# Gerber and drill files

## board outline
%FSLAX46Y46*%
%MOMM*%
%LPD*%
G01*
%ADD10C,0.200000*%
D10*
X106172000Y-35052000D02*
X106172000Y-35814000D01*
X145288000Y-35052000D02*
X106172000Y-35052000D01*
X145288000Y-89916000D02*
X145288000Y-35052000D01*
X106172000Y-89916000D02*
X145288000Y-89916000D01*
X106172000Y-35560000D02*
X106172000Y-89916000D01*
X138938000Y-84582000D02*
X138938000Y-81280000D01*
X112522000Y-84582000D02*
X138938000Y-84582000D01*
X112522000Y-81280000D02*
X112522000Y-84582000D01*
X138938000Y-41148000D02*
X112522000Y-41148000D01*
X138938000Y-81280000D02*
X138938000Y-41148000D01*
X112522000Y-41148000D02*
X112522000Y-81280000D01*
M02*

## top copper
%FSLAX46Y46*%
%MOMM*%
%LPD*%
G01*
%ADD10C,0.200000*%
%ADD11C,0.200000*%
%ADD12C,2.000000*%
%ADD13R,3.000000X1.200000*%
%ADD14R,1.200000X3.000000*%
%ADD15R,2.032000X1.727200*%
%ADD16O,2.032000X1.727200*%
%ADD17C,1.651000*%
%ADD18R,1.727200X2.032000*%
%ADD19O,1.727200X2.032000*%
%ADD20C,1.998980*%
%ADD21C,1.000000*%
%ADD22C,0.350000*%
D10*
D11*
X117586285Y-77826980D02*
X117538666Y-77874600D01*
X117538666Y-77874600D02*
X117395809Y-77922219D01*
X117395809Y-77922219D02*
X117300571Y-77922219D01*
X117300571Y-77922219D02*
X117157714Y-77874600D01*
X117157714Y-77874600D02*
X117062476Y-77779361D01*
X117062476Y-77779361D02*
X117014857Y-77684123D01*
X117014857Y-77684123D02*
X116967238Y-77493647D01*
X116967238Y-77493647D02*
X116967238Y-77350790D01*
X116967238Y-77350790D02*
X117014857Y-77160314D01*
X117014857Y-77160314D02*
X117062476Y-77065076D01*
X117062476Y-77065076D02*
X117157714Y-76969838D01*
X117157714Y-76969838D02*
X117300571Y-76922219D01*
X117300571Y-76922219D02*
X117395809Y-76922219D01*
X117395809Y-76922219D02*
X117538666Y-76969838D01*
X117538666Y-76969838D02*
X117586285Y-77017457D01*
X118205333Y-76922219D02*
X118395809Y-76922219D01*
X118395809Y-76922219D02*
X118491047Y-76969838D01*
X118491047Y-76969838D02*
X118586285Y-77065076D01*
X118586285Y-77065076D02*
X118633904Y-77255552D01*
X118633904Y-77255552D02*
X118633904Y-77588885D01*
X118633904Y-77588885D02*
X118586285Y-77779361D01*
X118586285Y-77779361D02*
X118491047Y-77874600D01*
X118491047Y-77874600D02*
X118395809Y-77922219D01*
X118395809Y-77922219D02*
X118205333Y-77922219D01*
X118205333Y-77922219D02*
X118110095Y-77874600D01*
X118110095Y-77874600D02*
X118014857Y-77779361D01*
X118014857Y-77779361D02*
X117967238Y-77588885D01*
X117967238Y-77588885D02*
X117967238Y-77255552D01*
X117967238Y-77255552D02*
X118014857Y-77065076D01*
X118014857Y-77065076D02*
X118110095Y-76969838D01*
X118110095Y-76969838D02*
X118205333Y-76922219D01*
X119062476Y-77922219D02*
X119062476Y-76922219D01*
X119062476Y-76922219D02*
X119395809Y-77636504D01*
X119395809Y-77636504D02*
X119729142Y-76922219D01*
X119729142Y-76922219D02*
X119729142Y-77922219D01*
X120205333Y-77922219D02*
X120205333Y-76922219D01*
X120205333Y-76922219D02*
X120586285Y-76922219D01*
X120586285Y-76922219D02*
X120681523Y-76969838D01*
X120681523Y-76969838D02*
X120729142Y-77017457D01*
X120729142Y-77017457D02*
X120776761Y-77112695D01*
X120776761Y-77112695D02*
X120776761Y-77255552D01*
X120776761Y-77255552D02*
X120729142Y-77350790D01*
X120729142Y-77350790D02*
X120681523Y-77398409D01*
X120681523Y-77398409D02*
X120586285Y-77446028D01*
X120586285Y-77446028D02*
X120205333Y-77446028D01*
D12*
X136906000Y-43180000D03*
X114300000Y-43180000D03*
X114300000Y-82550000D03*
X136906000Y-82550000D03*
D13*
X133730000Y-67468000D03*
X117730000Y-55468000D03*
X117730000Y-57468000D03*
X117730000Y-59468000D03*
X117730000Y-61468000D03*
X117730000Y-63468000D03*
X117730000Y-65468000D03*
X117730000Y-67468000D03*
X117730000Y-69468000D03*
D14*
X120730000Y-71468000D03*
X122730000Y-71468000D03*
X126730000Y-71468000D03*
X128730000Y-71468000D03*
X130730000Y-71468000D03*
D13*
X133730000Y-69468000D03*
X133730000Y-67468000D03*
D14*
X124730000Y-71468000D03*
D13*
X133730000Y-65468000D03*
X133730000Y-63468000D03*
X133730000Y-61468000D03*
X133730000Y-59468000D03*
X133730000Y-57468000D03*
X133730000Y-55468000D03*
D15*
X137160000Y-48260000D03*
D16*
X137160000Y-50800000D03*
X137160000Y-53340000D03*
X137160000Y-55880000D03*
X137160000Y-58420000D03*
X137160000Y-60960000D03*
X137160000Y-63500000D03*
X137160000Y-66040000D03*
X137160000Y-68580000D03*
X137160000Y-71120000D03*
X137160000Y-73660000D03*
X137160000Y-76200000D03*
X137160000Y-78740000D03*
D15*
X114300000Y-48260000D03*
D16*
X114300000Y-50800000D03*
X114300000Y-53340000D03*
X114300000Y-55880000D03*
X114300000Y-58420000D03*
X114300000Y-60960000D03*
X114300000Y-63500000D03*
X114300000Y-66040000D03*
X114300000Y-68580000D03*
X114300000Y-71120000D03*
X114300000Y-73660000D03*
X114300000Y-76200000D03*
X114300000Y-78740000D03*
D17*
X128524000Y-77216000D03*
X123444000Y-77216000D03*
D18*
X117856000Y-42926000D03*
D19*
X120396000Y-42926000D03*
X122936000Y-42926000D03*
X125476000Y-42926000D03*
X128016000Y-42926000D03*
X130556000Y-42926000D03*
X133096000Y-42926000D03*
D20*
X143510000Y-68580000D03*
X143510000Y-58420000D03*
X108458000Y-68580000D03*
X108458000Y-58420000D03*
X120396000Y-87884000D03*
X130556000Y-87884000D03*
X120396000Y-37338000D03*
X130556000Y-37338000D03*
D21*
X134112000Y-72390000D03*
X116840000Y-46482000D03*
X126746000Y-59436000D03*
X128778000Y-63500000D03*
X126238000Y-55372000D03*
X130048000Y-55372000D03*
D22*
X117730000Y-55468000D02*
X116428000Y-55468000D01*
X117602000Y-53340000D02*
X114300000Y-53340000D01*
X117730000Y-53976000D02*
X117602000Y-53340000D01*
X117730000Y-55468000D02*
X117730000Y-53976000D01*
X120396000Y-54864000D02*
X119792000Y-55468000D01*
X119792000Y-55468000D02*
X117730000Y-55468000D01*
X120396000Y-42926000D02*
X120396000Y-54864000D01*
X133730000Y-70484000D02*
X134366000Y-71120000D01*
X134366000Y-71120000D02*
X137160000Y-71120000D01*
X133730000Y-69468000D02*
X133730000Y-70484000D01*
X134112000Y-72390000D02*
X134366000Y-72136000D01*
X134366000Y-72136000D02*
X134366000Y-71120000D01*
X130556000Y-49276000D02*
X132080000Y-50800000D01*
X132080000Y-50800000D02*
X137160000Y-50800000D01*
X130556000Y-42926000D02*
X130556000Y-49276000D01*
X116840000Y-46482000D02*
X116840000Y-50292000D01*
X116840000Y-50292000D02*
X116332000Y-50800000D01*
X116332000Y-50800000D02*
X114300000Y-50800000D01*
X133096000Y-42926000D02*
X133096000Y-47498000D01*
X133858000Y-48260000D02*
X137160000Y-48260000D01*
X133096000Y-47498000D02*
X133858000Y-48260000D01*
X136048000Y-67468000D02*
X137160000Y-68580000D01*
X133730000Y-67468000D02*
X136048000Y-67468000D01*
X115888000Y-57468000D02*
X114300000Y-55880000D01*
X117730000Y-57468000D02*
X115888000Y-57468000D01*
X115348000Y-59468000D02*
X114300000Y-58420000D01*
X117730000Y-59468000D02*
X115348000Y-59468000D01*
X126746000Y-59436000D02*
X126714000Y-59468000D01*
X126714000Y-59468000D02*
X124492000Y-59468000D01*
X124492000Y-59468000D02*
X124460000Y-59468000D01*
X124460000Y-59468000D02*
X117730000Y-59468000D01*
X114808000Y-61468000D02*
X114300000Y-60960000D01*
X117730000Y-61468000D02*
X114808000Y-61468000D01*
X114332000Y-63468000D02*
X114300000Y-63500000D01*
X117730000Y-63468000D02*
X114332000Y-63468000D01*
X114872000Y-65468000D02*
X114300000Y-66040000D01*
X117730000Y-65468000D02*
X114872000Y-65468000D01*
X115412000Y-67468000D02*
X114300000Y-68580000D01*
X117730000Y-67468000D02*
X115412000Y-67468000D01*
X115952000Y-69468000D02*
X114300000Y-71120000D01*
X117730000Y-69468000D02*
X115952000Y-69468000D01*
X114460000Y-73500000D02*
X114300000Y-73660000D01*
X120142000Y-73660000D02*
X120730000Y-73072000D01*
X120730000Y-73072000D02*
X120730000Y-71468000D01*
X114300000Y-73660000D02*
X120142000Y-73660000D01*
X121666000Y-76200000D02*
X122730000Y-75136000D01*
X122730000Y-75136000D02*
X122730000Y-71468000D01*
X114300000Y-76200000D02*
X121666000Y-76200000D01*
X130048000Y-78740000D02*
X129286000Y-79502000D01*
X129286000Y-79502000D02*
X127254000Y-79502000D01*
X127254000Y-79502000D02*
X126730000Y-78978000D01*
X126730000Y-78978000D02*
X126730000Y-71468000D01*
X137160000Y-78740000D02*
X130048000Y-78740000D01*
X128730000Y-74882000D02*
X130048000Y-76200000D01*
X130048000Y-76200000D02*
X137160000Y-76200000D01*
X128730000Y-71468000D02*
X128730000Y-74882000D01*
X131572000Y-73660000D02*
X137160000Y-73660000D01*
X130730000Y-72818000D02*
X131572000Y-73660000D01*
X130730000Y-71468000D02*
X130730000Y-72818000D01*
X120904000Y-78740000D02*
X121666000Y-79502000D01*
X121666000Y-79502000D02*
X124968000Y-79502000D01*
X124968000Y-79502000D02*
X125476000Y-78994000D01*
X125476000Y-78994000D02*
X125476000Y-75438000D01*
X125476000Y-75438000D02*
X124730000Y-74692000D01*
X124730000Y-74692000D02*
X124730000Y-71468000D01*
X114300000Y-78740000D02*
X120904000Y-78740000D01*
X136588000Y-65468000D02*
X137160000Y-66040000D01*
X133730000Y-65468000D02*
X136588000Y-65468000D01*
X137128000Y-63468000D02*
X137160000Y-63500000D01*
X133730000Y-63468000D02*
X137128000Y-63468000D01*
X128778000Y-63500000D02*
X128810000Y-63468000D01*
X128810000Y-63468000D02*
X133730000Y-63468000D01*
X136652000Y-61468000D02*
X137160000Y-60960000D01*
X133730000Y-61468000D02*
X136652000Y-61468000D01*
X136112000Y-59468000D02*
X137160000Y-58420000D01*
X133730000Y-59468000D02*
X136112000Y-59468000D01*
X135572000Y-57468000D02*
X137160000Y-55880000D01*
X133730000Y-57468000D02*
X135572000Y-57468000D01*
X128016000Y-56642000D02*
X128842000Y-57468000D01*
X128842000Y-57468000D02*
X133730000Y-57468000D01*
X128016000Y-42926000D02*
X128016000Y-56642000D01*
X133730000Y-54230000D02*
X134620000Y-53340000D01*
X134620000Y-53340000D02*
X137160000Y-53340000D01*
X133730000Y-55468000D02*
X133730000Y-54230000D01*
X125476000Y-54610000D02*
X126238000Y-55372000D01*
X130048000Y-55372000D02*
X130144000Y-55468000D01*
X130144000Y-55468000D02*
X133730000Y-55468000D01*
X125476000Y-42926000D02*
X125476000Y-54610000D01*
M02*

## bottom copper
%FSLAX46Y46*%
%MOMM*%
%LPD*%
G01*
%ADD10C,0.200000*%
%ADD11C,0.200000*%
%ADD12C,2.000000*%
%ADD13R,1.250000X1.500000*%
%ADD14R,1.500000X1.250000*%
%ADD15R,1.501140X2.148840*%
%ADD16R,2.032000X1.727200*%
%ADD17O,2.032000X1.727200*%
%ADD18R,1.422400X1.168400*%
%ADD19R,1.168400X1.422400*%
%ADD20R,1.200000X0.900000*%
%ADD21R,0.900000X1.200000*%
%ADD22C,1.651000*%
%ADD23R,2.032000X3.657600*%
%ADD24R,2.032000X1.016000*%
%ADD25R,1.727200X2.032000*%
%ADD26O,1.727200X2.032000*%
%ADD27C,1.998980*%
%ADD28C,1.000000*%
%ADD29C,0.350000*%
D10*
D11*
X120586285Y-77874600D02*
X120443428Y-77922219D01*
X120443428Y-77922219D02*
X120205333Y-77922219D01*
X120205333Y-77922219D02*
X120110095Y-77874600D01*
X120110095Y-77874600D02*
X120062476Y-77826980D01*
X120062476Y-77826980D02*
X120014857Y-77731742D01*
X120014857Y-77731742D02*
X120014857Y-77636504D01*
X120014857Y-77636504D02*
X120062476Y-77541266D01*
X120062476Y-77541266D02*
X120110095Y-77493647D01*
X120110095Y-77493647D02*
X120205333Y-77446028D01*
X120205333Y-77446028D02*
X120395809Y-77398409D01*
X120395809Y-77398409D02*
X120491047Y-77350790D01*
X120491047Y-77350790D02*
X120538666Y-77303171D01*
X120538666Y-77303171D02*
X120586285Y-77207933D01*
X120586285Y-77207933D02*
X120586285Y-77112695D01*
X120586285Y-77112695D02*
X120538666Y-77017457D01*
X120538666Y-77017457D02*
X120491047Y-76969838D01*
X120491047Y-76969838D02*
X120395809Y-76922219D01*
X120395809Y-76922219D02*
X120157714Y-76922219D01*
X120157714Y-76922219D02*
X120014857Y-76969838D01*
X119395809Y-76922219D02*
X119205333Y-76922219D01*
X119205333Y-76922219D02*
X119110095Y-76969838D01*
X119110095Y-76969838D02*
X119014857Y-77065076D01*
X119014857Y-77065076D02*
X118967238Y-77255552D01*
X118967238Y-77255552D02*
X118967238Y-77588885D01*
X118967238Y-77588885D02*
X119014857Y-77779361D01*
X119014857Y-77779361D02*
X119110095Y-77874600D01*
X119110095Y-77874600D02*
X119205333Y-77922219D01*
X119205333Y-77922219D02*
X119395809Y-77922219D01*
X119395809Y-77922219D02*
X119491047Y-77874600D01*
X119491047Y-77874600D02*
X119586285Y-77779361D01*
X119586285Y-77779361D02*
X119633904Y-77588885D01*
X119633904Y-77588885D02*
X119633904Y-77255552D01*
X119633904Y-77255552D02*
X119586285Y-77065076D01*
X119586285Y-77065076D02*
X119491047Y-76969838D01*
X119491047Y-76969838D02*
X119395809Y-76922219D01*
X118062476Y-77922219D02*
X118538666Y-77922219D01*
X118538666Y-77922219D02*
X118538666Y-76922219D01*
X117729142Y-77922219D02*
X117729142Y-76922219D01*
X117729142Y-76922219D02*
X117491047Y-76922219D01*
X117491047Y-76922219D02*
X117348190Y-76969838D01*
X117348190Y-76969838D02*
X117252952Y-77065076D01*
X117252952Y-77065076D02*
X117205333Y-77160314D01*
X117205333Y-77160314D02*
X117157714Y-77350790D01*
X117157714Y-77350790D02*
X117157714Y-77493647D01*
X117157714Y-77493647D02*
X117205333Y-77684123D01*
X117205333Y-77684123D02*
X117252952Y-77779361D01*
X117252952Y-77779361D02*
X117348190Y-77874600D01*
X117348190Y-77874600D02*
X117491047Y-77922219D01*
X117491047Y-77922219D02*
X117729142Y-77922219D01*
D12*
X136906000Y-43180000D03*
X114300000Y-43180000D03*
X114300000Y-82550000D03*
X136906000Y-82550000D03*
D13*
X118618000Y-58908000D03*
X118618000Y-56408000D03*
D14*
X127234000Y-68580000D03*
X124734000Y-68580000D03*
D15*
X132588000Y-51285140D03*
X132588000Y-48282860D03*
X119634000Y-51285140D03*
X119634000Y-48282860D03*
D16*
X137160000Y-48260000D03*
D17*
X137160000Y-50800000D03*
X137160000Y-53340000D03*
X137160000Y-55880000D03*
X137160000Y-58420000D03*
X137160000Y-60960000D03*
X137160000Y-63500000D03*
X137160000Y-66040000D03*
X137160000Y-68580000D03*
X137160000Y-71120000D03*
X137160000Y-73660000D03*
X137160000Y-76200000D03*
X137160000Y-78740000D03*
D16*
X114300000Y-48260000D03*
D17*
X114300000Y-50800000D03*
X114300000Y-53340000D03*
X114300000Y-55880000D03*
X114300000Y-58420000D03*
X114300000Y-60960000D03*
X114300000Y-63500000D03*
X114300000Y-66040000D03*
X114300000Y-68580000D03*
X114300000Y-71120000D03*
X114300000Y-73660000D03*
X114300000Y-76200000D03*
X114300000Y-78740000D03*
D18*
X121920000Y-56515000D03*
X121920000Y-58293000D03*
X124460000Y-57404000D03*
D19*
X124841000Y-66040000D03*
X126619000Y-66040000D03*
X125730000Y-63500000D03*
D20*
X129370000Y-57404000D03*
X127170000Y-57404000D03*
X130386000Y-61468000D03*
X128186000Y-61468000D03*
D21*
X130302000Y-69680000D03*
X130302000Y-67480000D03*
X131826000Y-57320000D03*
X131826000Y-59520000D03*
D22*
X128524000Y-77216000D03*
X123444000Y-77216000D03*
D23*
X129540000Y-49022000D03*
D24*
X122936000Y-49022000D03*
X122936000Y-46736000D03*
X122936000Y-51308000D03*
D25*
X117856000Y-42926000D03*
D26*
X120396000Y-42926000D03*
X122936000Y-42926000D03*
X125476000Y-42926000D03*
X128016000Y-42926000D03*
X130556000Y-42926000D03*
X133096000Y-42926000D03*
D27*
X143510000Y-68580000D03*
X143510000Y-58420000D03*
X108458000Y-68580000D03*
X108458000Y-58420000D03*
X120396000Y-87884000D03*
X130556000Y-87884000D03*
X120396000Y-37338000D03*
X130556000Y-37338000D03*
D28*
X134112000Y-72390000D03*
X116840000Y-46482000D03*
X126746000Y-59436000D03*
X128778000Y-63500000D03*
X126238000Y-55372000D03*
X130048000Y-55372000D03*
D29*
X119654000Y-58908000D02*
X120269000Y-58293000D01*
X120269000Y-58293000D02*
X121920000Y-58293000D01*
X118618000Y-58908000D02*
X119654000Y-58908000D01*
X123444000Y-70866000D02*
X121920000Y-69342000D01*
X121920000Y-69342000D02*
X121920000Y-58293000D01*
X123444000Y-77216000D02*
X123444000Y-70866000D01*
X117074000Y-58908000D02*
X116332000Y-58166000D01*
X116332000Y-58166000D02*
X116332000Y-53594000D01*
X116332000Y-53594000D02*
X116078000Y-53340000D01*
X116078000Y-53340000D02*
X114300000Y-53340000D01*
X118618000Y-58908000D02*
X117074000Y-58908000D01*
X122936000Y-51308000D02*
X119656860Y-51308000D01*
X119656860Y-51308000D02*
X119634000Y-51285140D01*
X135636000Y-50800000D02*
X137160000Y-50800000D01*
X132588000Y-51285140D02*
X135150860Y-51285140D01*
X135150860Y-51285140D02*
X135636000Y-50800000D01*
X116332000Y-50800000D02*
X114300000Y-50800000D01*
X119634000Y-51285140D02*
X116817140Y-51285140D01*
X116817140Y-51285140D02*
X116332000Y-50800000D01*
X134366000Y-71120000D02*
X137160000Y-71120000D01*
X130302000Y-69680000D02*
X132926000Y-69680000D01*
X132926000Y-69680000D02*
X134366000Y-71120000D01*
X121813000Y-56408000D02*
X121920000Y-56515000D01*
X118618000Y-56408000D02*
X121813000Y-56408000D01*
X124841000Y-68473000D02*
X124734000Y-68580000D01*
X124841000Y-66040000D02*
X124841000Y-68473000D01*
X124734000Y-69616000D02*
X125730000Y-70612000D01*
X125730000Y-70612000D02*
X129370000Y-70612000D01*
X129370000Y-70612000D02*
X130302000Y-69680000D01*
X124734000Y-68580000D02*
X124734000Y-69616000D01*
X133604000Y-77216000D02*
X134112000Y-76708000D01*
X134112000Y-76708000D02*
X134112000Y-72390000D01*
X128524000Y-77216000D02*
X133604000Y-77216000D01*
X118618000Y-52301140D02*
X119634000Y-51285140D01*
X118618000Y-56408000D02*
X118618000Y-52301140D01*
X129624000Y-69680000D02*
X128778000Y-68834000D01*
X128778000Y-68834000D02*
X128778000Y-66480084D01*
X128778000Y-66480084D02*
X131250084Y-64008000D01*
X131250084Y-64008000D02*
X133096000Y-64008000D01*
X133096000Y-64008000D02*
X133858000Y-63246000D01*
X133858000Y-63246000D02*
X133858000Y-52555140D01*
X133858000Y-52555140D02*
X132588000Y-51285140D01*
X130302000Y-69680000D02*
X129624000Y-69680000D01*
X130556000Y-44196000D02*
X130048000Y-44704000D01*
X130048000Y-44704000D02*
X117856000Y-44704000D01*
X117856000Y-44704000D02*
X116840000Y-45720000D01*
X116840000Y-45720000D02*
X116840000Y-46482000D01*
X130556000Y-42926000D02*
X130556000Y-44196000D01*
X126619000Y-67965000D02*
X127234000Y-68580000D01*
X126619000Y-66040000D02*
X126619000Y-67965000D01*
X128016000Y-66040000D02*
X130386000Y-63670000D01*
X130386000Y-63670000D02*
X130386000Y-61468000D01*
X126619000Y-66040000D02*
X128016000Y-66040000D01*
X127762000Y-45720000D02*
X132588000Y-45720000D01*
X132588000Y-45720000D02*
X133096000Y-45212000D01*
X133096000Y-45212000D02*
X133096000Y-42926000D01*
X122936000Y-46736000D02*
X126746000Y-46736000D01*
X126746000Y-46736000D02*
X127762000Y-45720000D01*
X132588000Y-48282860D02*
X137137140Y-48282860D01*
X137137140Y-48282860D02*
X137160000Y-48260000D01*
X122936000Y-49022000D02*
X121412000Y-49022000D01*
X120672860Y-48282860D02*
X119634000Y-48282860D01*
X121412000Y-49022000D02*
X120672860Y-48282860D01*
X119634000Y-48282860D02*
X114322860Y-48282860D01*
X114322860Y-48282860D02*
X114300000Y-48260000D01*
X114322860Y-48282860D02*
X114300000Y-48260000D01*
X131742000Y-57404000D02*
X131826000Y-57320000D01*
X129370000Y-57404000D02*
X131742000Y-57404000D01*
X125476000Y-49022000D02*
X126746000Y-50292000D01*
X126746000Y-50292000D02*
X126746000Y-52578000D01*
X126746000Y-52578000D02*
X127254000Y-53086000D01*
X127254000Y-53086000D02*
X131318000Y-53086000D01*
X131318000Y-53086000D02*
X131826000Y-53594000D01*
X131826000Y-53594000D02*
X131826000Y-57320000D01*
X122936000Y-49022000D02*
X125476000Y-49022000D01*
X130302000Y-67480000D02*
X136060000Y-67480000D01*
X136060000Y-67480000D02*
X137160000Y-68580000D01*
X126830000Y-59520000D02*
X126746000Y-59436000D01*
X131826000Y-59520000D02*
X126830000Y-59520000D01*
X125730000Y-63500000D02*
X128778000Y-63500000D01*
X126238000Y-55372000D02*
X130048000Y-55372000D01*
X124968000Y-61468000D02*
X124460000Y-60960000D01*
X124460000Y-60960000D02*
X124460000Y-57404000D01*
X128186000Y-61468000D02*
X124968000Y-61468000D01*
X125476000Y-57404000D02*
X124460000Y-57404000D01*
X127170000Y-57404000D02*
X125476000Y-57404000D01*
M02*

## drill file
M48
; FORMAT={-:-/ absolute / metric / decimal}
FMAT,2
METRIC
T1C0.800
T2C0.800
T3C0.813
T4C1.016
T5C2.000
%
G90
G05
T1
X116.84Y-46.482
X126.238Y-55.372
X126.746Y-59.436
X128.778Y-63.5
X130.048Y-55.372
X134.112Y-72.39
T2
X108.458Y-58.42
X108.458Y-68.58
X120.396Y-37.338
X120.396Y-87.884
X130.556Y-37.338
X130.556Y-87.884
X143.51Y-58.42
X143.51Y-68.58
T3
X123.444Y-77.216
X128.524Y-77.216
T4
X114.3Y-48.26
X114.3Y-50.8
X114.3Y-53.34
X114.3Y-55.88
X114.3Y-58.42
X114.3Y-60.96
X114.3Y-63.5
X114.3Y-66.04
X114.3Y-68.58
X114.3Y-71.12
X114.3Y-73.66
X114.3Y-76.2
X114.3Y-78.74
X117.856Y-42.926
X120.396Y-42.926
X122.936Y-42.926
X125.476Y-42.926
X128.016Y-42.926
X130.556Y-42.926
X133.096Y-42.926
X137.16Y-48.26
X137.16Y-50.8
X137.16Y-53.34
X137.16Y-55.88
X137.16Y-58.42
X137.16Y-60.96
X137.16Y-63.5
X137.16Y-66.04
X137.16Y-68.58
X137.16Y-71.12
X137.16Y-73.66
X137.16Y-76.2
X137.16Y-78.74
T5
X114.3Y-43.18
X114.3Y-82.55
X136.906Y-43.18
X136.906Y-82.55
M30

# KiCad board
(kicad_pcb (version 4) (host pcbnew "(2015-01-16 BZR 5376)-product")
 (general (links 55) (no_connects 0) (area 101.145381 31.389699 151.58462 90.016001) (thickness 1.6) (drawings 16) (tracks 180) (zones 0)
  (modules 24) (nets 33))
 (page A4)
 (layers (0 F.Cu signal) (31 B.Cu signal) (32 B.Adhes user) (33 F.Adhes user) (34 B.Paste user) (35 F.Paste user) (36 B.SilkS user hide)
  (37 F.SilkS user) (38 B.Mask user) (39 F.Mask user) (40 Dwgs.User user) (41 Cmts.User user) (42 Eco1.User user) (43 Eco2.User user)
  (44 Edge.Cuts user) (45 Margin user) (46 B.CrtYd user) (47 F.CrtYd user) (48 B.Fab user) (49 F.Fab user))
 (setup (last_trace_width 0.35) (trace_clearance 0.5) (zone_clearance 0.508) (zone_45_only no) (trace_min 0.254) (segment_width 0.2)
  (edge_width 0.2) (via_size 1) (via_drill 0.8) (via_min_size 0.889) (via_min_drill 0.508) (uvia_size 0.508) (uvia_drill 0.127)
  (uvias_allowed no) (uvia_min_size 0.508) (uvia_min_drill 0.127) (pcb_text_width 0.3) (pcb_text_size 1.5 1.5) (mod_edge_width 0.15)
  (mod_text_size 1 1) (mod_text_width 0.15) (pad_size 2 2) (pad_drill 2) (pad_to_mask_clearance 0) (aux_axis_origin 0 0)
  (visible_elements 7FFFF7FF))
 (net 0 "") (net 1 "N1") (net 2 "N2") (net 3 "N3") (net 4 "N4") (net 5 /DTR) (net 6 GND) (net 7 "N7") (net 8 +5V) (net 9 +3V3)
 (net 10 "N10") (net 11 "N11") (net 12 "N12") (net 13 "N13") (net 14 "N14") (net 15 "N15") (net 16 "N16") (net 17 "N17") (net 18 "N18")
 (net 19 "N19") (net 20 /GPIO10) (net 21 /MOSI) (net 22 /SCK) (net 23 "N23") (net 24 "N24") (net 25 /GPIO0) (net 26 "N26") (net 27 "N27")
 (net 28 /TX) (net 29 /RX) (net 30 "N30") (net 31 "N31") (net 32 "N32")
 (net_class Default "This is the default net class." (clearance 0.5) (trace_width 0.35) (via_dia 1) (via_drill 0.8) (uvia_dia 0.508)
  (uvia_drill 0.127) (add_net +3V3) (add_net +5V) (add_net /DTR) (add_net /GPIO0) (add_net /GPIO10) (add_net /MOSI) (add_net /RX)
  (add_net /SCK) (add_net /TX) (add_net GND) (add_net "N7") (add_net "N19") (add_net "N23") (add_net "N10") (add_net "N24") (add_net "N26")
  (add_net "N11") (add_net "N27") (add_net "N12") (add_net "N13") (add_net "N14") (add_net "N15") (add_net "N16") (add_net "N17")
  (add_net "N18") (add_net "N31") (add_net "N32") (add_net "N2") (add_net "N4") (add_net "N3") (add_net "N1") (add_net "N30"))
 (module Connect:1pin (layer F.Cu) (at 136.906 43.18)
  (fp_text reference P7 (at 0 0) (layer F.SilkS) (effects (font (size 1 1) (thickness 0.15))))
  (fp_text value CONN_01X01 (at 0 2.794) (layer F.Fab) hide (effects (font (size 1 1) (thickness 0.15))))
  (pad 1 thru_hole circle (at 0 0) (size 2 2) (drill 2) (layers *.Cu *.Mask F.SilkS) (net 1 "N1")))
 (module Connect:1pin (layer F.Cu) (at 114.3 43.18)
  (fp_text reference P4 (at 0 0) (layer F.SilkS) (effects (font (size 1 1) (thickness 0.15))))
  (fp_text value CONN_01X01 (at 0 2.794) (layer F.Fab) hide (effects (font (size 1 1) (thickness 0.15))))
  (pad 1 thru_hole circle (at 0 0) (size 2 2) (drill 2) (layers *.Cu *.Mask F.SilkS) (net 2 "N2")))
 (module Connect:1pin (layer F.Cu) (at 114.3 82.55)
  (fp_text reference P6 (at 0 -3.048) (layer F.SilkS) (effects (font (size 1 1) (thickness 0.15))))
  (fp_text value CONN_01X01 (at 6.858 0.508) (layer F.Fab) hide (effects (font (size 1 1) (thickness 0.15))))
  (pad 1 thru_hole circle (at 0 0) (size 2 2) (drill 2) (layers *.Cu *.Mask F.SilkS) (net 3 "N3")))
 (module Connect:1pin (layer F.Cu) (at 136.906 82.55)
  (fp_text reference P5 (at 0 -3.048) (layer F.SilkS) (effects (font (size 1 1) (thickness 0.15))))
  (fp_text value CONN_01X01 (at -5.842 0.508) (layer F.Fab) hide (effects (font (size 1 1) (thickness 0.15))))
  (pad 1 thru_hole circle (at 0 0) (size 2 2) (drill 2) (layers *.Cu *.Mask F.SilkS) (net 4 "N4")))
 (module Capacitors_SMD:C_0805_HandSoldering (layer B.Cu) (at 118.618 57.658 90)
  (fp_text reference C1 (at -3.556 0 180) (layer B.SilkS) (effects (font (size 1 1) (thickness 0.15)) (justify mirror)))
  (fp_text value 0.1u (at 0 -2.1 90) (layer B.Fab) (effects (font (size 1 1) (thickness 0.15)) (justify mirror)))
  (pad 1 smd rect (at -1.25 0 90) (size 1.5 1.25) (layers B.Cu B.Paste B.Mask) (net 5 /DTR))
  (pad 2 smd rect (at 1.25 0 90) (size 1.5 1.25) (layers B.Cu B.Paste B.Mask) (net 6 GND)))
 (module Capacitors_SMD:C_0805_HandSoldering (layer B.Cu) (at 125.984 68.58 180)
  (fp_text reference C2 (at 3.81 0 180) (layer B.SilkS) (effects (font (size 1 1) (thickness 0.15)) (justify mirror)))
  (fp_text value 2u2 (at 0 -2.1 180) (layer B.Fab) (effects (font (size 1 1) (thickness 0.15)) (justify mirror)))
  (pad 1 smd rect (at -1.25 0 180) (size 1.5 1.25) (layers B.Cu B.Paste B.Mask) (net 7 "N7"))
  (pad 2 smd rect (at 1.25 0 180) (size 1.5 1.25) (layers B.Cu B.Paste B.Mask) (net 6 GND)))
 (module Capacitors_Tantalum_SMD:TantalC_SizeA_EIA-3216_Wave (layer B.Cu) (at 132.588 49.784 270)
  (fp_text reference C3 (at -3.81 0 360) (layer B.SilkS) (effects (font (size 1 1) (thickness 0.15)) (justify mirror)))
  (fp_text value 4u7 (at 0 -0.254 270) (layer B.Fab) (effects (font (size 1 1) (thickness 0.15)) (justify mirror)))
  (pad 2 smd rect (at 1.50114 0 270) (size 2.14884 1.50114) (layers B.Cu B.Paste B.Mask) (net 6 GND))
  (pad 1 smd rect (at -1.50114 0 270) (size 2.14884 1.50114) (layers B.Cu B.Paste B.Mask) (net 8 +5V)))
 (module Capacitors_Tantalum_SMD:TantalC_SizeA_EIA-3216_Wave (layer B.Cu) (at 119.634 49.784 270)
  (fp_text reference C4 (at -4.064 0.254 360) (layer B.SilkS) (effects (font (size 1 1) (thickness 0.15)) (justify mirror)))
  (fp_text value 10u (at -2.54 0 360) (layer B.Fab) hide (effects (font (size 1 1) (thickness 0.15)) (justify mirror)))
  (pad 2 smd rect (at 1.50114 0 270) (size 2.14884 1.50114) (layers B.Cu B.Paste B.Mask) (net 6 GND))
  (pad 1 smd rect (at -1.50114 0 270) (size 2.14884 1.50114) (layers B.Cu B.Paste B.Mask) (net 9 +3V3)))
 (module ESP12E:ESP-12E (layer F.Cu) (at 125.73 61.468 270)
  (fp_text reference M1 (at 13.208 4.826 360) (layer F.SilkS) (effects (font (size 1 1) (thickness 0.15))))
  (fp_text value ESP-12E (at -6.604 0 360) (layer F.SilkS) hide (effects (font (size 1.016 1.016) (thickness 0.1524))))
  (pad 16 smd rect (at 6 -8 270) (size 1.2 3) (layers F.Cu F.Paste F.Mask) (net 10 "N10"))
  (pad 1 smd rect (at -6 8 270) (size 1.2 3) (layers F.Cu F.Paste F.Mask) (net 5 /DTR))
  (pad 2 smd rect (at -4 8 270) (size 1.2 3) (layers F.Cu F.Paste F.Mask) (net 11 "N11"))
  (pad 3 smd rect (at -2 8 270) (size 1.2 3) (layers F.Cu F.Paste F.Mask) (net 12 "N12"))
  (pad 4 smd rect (at 0 8 270) (size 1.2 3) (layers F.Cu F.Paste F.Mask) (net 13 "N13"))
  (pad 5 smd rect (at 2 8 270) (size 1.2 3) (layers F.Cu F.Paste F.Mask) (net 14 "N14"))
  (pad 6 smd rect (at 4 8 270) (size 1.2 3) (layers F.Cu F.Paste F.Mask) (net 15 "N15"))
  (pad 7 smd rect (at 6 8 270) (size 1.2 3) (layers F.Cu F.Paste F.Mask) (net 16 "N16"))
  (pad 8 smd rect (at 8 8 270) (size 1.2 3) (layers F.Cu F.Paste F.Mask) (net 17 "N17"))
  (pad 9 smd rect (at 10 5 180) (size 1.2 3) (layers F.Cu F.Paste F.Mask) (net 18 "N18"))
  (pad 10 smd rect (at 10 3 180) (size 1.2 3) (layers F.Cu F.Paste F.Mask) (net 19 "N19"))
  (pad 12 smd rect (at 10 -1 180) (size 1.2 3) (layers F.Cu F.Paste F.Mask) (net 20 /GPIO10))
  (pad 13 smd rect (at 10 -3 180) (size 1.2 3) (layers F.Cu F.Paste F.Mask) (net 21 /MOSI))
  (pad 14 smd rect (at 10 -5 180) (size 1.2 3) (layers F.Cu F.Paste F.Mask) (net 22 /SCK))
  (pad 15 smd rect (at 8 -8 270) (size 1.2 3) (layers F.Cu F.Paste F.Mask) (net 6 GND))
  (pad 16 smd rect (at 6 -8 270) (size 1.2 3) (layers F.Cu F.Paste F.Mask) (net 10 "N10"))
  (pad 11 smd rect (at 10 1 180) (size 1.2 3) (layers F.Cu F.Paste F.Mask) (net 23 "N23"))
  (pad 17 smd rect (at 4 -8 270) (size 1.2 3) (layers F.Cu F.Paste F.Mask) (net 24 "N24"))
  (pad 18 smd rect (at 2 -8 270) (size 1.2 3) (layers F.Cu F.Paste F.Mask) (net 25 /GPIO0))
  (pad 19 smd rect (at 0 -8 270) (size 1.2 3) (layers F.Cu F.Paste F.Mask) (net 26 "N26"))
  (pad 20 smd rect (at -2 -8 270) (size 1.2 3) (layers F.Cu F.Paste F.Mask) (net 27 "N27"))
  (pad 21 smd rect (at -4 -8 270) (size 1.2 3) (layers F.Cu F.Paste F.Mask) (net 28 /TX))
  (pad 22 smd rect (at -6 -8 270) (size 1.2 3) (layers F.Cu F.Paste F.Mask) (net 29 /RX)))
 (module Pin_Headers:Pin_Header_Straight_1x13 (layer F.Cu) (at 137.16 48.26)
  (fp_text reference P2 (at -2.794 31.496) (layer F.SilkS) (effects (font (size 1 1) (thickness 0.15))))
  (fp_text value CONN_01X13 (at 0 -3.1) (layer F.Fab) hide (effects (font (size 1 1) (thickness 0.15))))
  (pad 1 thru_hole rect (at 0 0) (size 2.032 1.7272) (drill 1.016) (layers *.Cu *.Mask F.SilkS) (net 8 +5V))
  (pad 2 thru_hole oval (at 0 2.54) (size 2.032 1.7272) (drill 1.016) (layers *.Cu *.Mask F.SilkS) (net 6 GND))
  (pad 3 thru_hole oval (at 0 5.08) (size 2.032 1.7272) (drill 1.016) (layers *.Cu *.Mask F.SilkS) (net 29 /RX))
  (pad 4 thru_hole oval (at 0 7.62) (size 2.032 1.7272) (drill 1.016) (layers *.Cu *.Mask F.SilkS) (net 28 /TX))
  (pad 5 thru_hole oval (at 0 10.16) (size 2.032 1.7272) (drill 1.016) (layers *.Cu *.Mask F.SilkS) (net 27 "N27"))
  (pad 6 thru_hole oval (at 0 12.7) (size 2.032 1.7272) (drill 1.016) (layers *.Cu *.Mask F.SilkS) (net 26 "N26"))
  (pad 7 thru_hole oval (at 0 15.24) (size 2.032 1.7272) (drill 1.016) (layers *.Cu *.Mask F.SilkS) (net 25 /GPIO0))
  (pad 8 thru_hole oval (at 0 17.78) (size 2.032 1.7272) (drill 1.016) (layers *.Cu *.Mask F.SilkS) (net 24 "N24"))
  (pad 9 thru_hole oval (at 0 20.32) (size 2.032 1.7272) (drill 1.016) (layers *.Cu *.Mask F.SilkS) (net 10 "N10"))
  (pad 10 thru_hole oval (at 0 22.86) (size 2.032 1.7272) (drill 1.016) (layers *.Cu *.Mask F.SilkS) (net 6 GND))
  (pad 11 thru_hole oval (at 0 25.4) (size 2.032 1.7272) (drill 1.016) (layers *.Cu *.Mask F.SilkS) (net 22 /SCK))
  (pad 12 thru_hole oval (at 0 27.94) (size 2.032 1.7272) (drill 1.016) (layers *.Cu *.Mask F.SilkS) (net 21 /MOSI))
  (pad 13 thru_hole oval (at 0 30.48) (size 2.032 1.7272) (drill 1.016) (layers *.Cu *.Mask F.SilkS) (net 20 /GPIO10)))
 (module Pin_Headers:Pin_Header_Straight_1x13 (layer F.Cu) (at 114.3 48.26)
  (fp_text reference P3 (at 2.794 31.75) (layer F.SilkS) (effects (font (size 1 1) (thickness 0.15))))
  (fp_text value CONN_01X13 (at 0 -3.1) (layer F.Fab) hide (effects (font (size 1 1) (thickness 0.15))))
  (pad 1 thru_hole rect (at 0 0) (size 2.032 1.7272) (drill 1.016) (layers *.Cu *.Mask F.SilkS) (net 9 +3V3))
  (pad 2 thru_hole oval (at 0 2.54) (size 2.032 1.7272) (drill 1.016) (layers *.Cu *.Mask F.SilkS) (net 6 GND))
  (pad 3 thru_hole oval (at 0 5.08) (size 2.032 1.7272) (drill 1.016) (layers *.Cu *.Mask F.SilkS) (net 5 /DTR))
  (pad 4 thru_hole oval (at 0 7.62) (size 2.032 1.7272) (drill 1.016) (layers *.Cu *.Mask F.SilkS) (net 11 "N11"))
  (pad 5 thru_hole oval (at 0 10.16) (size 2.032 1.7272) (drill 1.016) (layers *.Cu *.Mask F.SilkS) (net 12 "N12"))
  (pad 6 thru_hole oval (at 0 12.7) (size 2.032 1.7272) (drill 1.016) (layers *.Cu *.Mask F.SilkS) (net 13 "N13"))
  (pad 7 thru_hole oval (at 0 15.24) (size 2.032 1.7272) (drill 1.016) (layers *.Cu *.Mask F.SilkS) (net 14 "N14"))
  (pad 8 thru_hole oval (at 0 17.78) (size 2.032 1.7272) (drill 1.016) (layers *.Cu *.Mask F.SilkS) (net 15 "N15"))
  (pad 9 thru_hole oval (at 0 20.32) (size 2.032 1.7272) (drill 1.016) (layers *.Cu *.Mask F.SilkS) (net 16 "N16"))
  (pad 10 thru_hole oval (at 0 22.86) (size 2.032 1.7272) (drill 1.016) (layers *.Cu *.Mask F.SilkS) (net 17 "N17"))
  (pad 11 thru_hole oval (at 0 25.4) (size 2.032 1.7272) (drill 1.016) (layers *.Cu *.Mask F.SilkS) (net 18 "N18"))
  (pad 12 thru_hole oval (at 0 27.94) (size 2.032 1.7272) (drill 1.016) (layers *.Cu *.Mask F.SilkS) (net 19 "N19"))
  (pad 13 thru_hole oval (at 0 30.48) (size 2.032 1.7272) (drill 1.016) (layers *.Cu *.Mask F.SilkS) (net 23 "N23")))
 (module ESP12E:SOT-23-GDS (layer B.Cu) (at 123.19 57.404 270)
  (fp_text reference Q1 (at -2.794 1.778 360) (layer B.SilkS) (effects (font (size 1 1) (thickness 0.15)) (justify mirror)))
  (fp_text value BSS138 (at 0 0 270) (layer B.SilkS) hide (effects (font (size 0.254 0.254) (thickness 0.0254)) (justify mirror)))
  (pad S smd rect (at -0.889 1.27 270) (size 1.1684 1.4224) (layers B.Cu B.Paste B.Mask) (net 6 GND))
  (pad G smd rect (at 0.889 1.27 270) (size 1.1684 1.4224) (layers B.Cu B.Paste B.Mask) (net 5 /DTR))
  (pad D smd rect (at 0 -1.27 270) (size 1.1684 1.4224) (layers B.Cu B.Paste B.Mask) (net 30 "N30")))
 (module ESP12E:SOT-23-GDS (layer B.Cu) (at 125.73 64.77)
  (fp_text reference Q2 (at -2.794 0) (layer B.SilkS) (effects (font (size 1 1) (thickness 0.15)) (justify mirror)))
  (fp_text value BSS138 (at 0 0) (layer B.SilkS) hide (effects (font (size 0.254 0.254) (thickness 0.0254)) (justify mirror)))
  (pad S smd rect (at -0.889 1.27) (size 1.1684 1.4224) (layers B.Cu B.Paste B.Mask) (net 6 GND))
  (pad G smd rect (at 0.889 1.27) (size 1.1684 1.4224) (layers B.Cu B.Paste B.Mask) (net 7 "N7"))
  (pad D smd rect (at 0 -1.27) (size 1.1684 1.4224) (layers B.Cu B.Paste B.Mask) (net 25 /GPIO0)))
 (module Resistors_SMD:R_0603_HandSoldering (layer B.Cu) (at 128.27 57.404 180)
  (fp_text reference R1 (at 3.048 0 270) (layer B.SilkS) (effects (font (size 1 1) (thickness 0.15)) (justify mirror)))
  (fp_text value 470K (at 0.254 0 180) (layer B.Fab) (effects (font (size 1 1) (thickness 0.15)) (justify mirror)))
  (pad 1 smd rect (at -1.1 0 180) (size 1.2 0.9) (layers B.Cu B.Paste B.Mask) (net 9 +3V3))
  (pad 2 smd rect (at 1.1 0 180) (size 1.2 0.9) (layers B.Cu B.Paste B.Mask) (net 30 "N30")))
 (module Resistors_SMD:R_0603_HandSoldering (layer B.Cu) (at 129.286 61.468 180)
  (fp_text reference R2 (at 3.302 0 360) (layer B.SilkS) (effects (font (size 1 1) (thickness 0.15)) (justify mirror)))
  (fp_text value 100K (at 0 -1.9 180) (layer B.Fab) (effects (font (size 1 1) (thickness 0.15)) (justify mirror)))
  (pad 1 smd rect (at -1.1 0 180) (size 1.2 0.9) (layers B.Cu B.Paste B.Mask) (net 7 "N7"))
  (pad 2 smd rect (at 1.1 0 180) (size 1.2 0.9) (layers B.Cu B.Paste B.Mask) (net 30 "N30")))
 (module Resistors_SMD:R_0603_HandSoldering (layer B.Cu) (at 130.302 68.58 90)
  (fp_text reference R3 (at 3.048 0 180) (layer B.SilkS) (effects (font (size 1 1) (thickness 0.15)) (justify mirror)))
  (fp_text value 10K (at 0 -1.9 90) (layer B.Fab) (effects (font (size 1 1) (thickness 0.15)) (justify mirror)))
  (pad 1 smd rect (at -1.1 0 90) (size 1.2 0.9) (layers B.Cu B.Paste B.Mask) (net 6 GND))
  (pad 2 smd rect (at 1.1 0 90) (size 1.2 0.9) (layers B.Cu B.Paste B.Mask) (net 10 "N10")))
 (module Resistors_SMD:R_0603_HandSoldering (layer B.Cu) (at 131.826 58.42 270)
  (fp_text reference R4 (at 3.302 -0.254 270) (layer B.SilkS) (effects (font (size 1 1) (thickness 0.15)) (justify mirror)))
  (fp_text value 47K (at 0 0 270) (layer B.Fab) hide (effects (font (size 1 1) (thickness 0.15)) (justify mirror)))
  (pad 1 smd rect (at -1.1 0 270) (size 1.2 0.9) (layers B.Cu B.Paste B.Mask) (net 9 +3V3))
  (pad 2 smd rect (at 1.1 0 270) (size 1.2 0.9) (layers B.Cu B.Paste B.Mask) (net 12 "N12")))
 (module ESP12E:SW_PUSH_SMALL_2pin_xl (layer F.Cu) (at 125.984 77.216 180)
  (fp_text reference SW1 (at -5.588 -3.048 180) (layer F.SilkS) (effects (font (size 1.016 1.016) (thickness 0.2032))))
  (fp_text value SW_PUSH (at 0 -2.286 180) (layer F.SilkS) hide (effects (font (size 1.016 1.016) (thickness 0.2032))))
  (pad 1 thru_hole circle (at -2.54 0 180) (size 1.651 1.651) (drill 0.8128) (layers *.Cu *.Mask F.SilkS) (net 6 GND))
  (pad 2 thru_hole circle (at 2.54 0 180) (size 1.651 1.651) (drill 0.8128) (layers *.Cu *.Mask F.SilkS) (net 5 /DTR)))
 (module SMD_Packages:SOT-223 (layer B.Cu) (at 126.238 49.022 90)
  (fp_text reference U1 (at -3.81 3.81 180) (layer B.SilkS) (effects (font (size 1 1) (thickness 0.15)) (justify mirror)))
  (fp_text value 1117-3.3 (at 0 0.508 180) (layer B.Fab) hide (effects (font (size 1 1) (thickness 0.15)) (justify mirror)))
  (pad 4 smd rect (at 0 3.302 90) (size 3.6576 2.032) (layers B.Cu B.Paste B.Mask))
  (pad 2 smd rect (at 0 -3.302 90) (size 1.016 2.032) (layers B.Cu B.Paste B.Mask) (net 9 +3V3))
  (pad 3 smd rect (at 2.286 -3.302 90) (size 1.016 2.032) (layers B.Cu B.Paste B.Mask) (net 8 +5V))
  (pad 1 smd rect (at -2.286 -3.302 90) (size 1.016 2.032) (layers B.Cu B.Paste B.Mask) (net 6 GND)))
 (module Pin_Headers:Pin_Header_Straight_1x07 (layer F.Cu) (at 117.856 42.926 90)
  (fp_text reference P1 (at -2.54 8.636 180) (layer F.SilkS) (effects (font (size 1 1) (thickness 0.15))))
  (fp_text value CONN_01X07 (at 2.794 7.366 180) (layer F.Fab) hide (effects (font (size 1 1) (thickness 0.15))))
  (pad 1 thru_hole rect (at 0 0 90) (size 2.032 1.7272) (drill 1.016) (layers *.Cu *.Mask F.SilkS) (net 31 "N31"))
  (pad 2 thru_hole oval (at 0 2.54 90) (size 2.032 1.7272) (drill 1.016) (layers *.Cu *.Mask F.SilkS) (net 5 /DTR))
  (pad 3 thru_hole oval (at 0 5.08 90) (size 2.032 1.7272) (drill 1.016) (layers *.Cu *.Mask F.SilkS) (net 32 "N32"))
  (pad 4 thru_hole oval (at 0 7.62 90) (size 2.032 1.7272) (drill 1.016) (layers *.Cu *.Mask F.SilkS) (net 29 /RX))
  (pad 5 thru_hole oval (at 0 10.16 90) (size 2.032 1.7272) (drill 1.016) (layers *.Cu *.Mask F.SilkS) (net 28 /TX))
  (pad 6 thru_hole oval (at 0 12.7 90) (size 2.032 1.7272) (drill 1.016) (layers *.Cu *.Mask F.SilkS) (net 6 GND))
  (pad 7 thru_hole oval (at 0 15.24 90) (size 2.032 1.7272) (drill 1.016) (layers *.Cu *.Mask F.SilkS) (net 8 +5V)))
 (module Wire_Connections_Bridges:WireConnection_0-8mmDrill (layer F.Cu) (at 143.51 63.5 90)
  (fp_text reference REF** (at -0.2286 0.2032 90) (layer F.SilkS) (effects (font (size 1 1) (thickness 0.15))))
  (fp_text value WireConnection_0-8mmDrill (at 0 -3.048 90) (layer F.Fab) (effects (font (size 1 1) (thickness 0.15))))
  (pad 1 thru_hole circle (at -5.08 0 90) (size 1.99898 1.99898) (drill 0.8001) (layers *.Cu *.Mask F.SilkS))
  (pad 2 thru_hole circle (at 5.08 0 90) (size 1.99898 1.99898) (drill 0.8001) (layers *.Cu *.Mask F.SilkS)))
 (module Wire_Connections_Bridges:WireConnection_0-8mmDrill (layer F.Cu) (at 108.458 63.5 90)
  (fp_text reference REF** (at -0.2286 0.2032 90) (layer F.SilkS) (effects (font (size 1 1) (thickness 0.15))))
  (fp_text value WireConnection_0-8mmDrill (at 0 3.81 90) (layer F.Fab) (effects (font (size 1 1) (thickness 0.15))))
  (pad 1 thru_hole circle (at -5.08 0 90) (size 1.99898 1.99898) (drill 0.8001) (layers *.Cu *.Mask F.SilkS))
  (pad 2 thru_hole circle (at 5.08 0 90) (size 1.99898 1.99898) (drill 0.8001) (layers *.Cu *.Mask F.SilkS)))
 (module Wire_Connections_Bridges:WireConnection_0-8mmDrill (layer F.Cu) (at 125.476 87.884)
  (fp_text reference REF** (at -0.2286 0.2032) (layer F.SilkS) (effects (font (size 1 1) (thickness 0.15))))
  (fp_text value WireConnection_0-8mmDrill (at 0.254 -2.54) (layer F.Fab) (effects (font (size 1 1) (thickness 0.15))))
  (pad 1 thru_hole circle (at -5.08 0) (size 1.99898 1.99898) (drill 0.8001) (layers *.Cu *.Mask F.SilkS))
  (pad 2 thru_hole circle (at 5.08 0) (size 1.99898 1.99898) (drill 0.8001) (layers *.Cu *.Mask F.SilkS)))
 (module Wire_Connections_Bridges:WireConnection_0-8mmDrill (layer F.Cu) (at 125.476 37.338)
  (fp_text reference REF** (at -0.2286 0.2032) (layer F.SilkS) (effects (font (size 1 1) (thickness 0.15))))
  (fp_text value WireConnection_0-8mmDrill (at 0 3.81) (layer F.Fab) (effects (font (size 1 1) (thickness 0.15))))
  (pad 1 thru_hole circle (at -5.08 0) (size 1.99898 1.99898) (drill 0.8001) (layers *.Cu *.Mask F.SilkS))
  (pad 2 thru_hole circle (at 5.08 0) (size 1.99898 1.99898) (drill 0.8001) (layers *.Cu *.Mask F.SilkS)))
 (gr_line (start 106.172 35.052) (end 106.172 35.814) (angle 90) (layer Edge.Cuts) (width 0.2))
 (gr_line (start 145.288 35.052) (end 106.172 35.052) (angle 90) (layer Edge.Cuts) (width 0.2))
 (gr_line (start 145.288 89.916) (end 145.288 35.052) (angle 90) (layer Edge.Cuts) (width 0.2))
 (gr_line (start 106.172 89.916) (end 145.288 89.916) (angle 90) (layer Edge.Cuts) (width 0.2))
 (gr_line (start 106.172 35.56) (end 106.172 89.916) (angle 90) (layer Edge.Cuts) (width 0.2))
 (gr_line (start 138.938 84.582) (end 138.938 81.28) (angle 90) (layer Edge.Cuts) (width 0.2))
 (gr_line (start 112.522 84.582) (end 138.938 84.582) (angle 90) (layer Edge.Cuts) (width 0.2))
 (gr_line (start 112.522 81.28) (end 112.522 84.582) (angle 90) (layer Edge.Cuts) (width 0.2))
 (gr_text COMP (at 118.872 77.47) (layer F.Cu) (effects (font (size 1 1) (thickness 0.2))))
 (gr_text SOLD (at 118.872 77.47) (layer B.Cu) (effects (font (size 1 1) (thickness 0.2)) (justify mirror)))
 (gr_line (start 138.938 41.148) (end 112.522 41.148) (angle 90) (layer Edge.Cuts) (width 0.2))
 (gr_line (start 138.938 81.28) (end 138.938 41.148) (angle 90) (layer Edge.Cuts) (width 0.2))
 (gr_line (start 112.522 41.148) (end 112.522 81.28) (angle 90) (layer Edge.Cuts) (width 0.2))
 (segment (start 117.73 55.468) (end 116.428 55.468) (width 0.35) (layer F.Cu) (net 5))
 (segment (start 117.602 53.34) (end 114.3 53.34) (width 0.35) (layer F.Cu) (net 5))
 (segment (start 117.73 53.976) (end 117.602 53.34) (width 0.35) (layer F.Cu) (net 5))
 (segment (start 117.73 55.468) (end 117.73 53.976) (width 0.35) (layer F.Cu) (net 5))
 (segment (start 120.396 54.864) (end 119.792 55.468) (width 0.35) (layer F.Cu) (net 5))
 (segment (start 119.792 55.468) (end 117.73 55.468) (width 0.35) (layer F.Cu) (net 5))
 (segment (start 120.396 42.926) (end 120.396 54.864) (width 0.35) (layer F.Cu) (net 5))
 (segment (start 119.654 58.908) (end 120.269 58.293) (width 0.35) (layer B.Cu) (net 5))
 (segment (start 120.269 58.293) (end 121.92 58.293) (width 0.35) (layer B.Cu) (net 5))
 (segment (start 118.618 58.908) (end 119.654 58.908) (width 0.35) (layer B.Cu) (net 5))
 (segment (start 123.444 70.866) (end 121.92 69.342) (width 0.35) (layer B.Cu) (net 5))
 (segment (start 121.92 69.342) (end 121.92 58.293) (width 0.35) (layer B.Cu) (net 5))
 (segment (start 123.444 77.216) (end 123.444 70.866) (width 0.35) (layer B.Cu) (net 5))
 (segment (start 117.074 58.908) (end 116.332 58.166) (width 0.35) (layer B.Cu) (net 5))
 (segment (start 116.332 58.166) (end 116.332 53.594) (width 0.35) (layer B.Cu) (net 5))
 (segment (start 116.332 53.594) (end 116.078 53.34) (width 0.35) (layer B.Cu) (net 5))
 (segment (start 116.078 53.34) (end 114.3 53.34) (width 0.35) (layer B.Cu) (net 5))
 (segment (start 118.618 58.908) (end 117.074 58.908) (width 0.35) (layer B.Cu) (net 5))
 (segment (start 122.936 51.308) (end 119.65686 51.308) (width 0.35) (layer B.Cu) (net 6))
 (segment (start 119.65686 51.308) (end 119.634 51.28514) (width 0.35) (layer B.Cu) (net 6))
 (segment (start 135.636 50.8) (end 137.16 50.8) (width 0.35) (layer B.Cu) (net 6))
 (segment (start 132.588 51.28514) (end 135.15086 51.28514) (width 0.35) (layer B.Cu) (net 6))
 (segment (start 135.15086 51.28514) (end 135.636 50.8) (width 0.35) (layer B.Cu) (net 6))
 (segment (start 116.332 50.8) (end 114.3 50.8) (width 0.35) (layer B.Cu) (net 6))
 (segment (start 119.634 51.28514) (end 116.81714 51.28514) (width 0.35) (layer B.Cu) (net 6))
 (segment (start 116.81714 51.28514) (end 116.332 50.8) (width 0.35) (layer B.Cu) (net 6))
 (segment (start 134.366 71.12) (end 137.16 71.12) (width 0.35) (layer B.Cu) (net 6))
 (segment (start 130.302 69.68) (end 132.926 69.68) (width 0.35) (layer B.Cu) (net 6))
 (segment (start 132.926 69.68) (end 134.366 71.12) (width 0.35) (layer B.Cu) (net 6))
 (segment (start 133.73 70.484) (end 134.366 71.12) (width 0.35) (layer F.Cu) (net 6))
 (segment (start 134.366 71.12) (end 137.16 71.12) (width 0.35) (layer F.Cu) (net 6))
 (segment (start 133.73 69.468) (end 133.73 70.484) (width 0.35) (layer F.Cu) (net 6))
 (via (at 134.112 72.39) (size 1) (layers F.Cu B.Cu) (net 6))
 (segment (start 134.112 72.39) (end 134.366 72.136) (width 0.35) (layer F.Cu) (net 6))
 (segment (start 134.366 72.136) (end 134.366 71.12) (width 0.35) (layer F.Cu) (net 6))
 (segment (start 130.556 49.276) (end 132.08 50.8) (width 0.35) (layer F.Cu) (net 6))
 (segment (start 132.08 50.8) (end 137.16 50.8) (width 0.35) (layer F.Cu) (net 6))
 (segment (start 130.556 42.926) (end 130.556 49.276) (width 0.35) (layer F.Cu) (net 6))
 (segment (start 121.813 56.408) (end 121.92 56.515) (width 0.35) (layer B.Cu) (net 6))
 (segment (start 118.618 56.408) (end 121.813 56.408) (width 0.35) (layer B.Cu) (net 6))
 (segment (start 124.841 68.473) (end 124.734 68.58) (width 0.35) (layer B.Cu) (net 6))
 (segment (start 124.841 66.04) (end 124.841 68.473) (width 0.35) (layer B.Cu) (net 6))
 (segment (start 124.734 69.616) (end 125.73 70.612) (width 0.35) (layer B.Cu) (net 6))
 (segment (start 125.73 70.612) (end 129.37 70.612) (width 0.35) (layer B.Cu) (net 6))
 (segment (start 129.37 70.612) (end 130.302 69.68) (width 0.35) (layer B.Cu) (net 6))
 (segment (start 124.734 68.58) (end 124.734 69.616) (width 0.35) (layer B.Cu) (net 6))
 (segment (start 133.604 77.216) (end 134.112 76.708) (width 0.35) (layer B.Cu) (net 6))
 (segment (start 134.112 76.708) (end 134.112 72.39) (width 0.35) (layer B.Cu) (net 6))
 (segment (start 128.524 77.216) (end 133.604 77.216) (width 0.35) (layer B.Cu) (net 6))
 (segment (start 118.618 52.30114) (end 119.634 51.28514) (width 0.35) (layer B.Cu) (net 6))
 (segment (start 118.618 56.408) (end 118.618 52.30114) (width 0.35) (layer B.Cu) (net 6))
 (segment (start 129.624 69.68) (end 128.778 68.834) (width 0.35) (layer B.Cu) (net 6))
 (segment (start 128.778 68.834) (end 128.778 66.480084) (width 0.35) (layer B.Cu) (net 6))
 (segment (start 128.778 66.480084) (end 131.250084 64.008) (width 0.35) (layer B.Cu) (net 6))
 (segment (start 131.250084 64.008) (end 133.096 64.008) (width 0.35) (layer B.Cu) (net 6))
 (segment (start 133.096 64.008) (end 133.858 63.246) (width 0.35) (layer B.Cu) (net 6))
 (segment (start 133.858 63.246) (end 133.858 52.55514) (width 0.35) (layer B.Cu) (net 6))
 (segment (start 133.858 52.55514) (end 132.588 51.28514) (width 0.35) (layer B.Cu) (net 6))
 (segment (start 130.302 69.68) (end 129.624 69.68) (width 0.35) (layer B.Cu) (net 6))
 (segment (start 130.556 44.196) (end 130.048 44.704) (width 0.35) (layer B.Cu) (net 6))
 (segment (start 130.048 44.704) (end 117.856 44.704) (width 0.35) (layer B.Cu) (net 6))
 (segment (start 117.856 44.704) (end 116.84 45.72) (width 0.35) (layer B.Cu) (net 6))
 (segment (start 116.84 45.72) (end 116.84 46.482) (width 0.35) (layer B.Cu) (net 6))
 (via (at 116.84 46.482) (size 1) (layers F.Cu B.Cu) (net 6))
 (segment (start 116.84 46.482) (end 116.84 50.292) (width 0.35) (layer F.Cu) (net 6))
 (segment (start 116.84 50.292) (end 116.332 50.8) (width 0.35) (layer F.Cu) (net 6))
 (segment (start 116.332 50.8) (end 114.3 50.8) (width 0.35) (layer F.Cu) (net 6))
 (segment (start 130.556 42.926) (end 130.556 44.196) (width 0.35) (layer B.Cu) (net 6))
 (segment (start 126.619 67.965) (end 127.234 68.58) (width 0.35) (layer B.Cu) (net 7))
 (segment (start 126.619 66.04) (end 126.619 67.965) (width 0.35) (layer B.Cu) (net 7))
 (segment (start 128.016 66.04) (end 130.386 63.67) (width 0.35) (layer B.Cu) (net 7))
 (segment (start 130.386 63.67) (end 130.386 61.468) (width 0.35) (layer B.Cu) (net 7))
 (segment (start 126.619 66.04) (end 128.016 66.04) (width 0.35) (layer B.Cu) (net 7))
 (segment (start 133.096 42.926) (end 133.096 47.498) (width 0.35) (layer F.Cu) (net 8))
 (segment (start 133.858 48.26) (end 137.16 48.26) (width 0.35) (layer F.Cu) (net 8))
 (segment (start 133.096 47.498) (end 133.858 48.26) (width 0.35) (layer F.Cu) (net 8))
 (segment (start 127.762 45.72) (end 132.588 45.72) (width 0.35) (layer B.Cu) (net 8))
 (segment (start 132.588 45.72) (end 133.096 45.212) (width 0.35) (layer B.Cu) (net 8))
 (segment (start 133.096 45.212) (end 133.096 42.926) (width 0.35) (layer B.Cu) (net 8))
 (segment (start 122.936 46.736) (end 126.746 46.736) (width 0.35) (layer B.Cu) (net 8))
 (segment (start 126.746 46.736) (end 127.762 45.72) (width 0.35) (layer B.Cu) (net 8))
 (segment (start 132.588 48.28286) (end 137.13714 48.28286) (width 0.35) (layer B.Cu) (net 8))
 (segment (start 137.13714 48.28286) (end 137.16 48.26) (width 0.35) (layer B.Cu) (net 8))
 (segment (start 122.936 49.022) (end 121.412 49.022) (width 0.35) (layer B.Cu) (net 9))
 (segment (start 120.67286 48.28286) (end 119.634 48.28286) (width 0.35) (layer B.Cu) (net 9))
 (segment (start 121.412 49.022) (end 120.67286 48.28286) (width 0.35) (layer B.Cu) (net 9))
 (segment (start 119.634 48.28286) (end 114.32286 48.28286) (width 0.35) (layer B.Cu) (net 9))
 (segment (start 114.32286 48.28286) (end 114.3 48.26) (width 0.35) (layer B.Cu) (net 9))
 (segment (start 114.32286 48.28286) (end 114.3 48.26) (width 0.35) (layer B.Cu) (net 9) (status 30))
 (segment (start 131.742 57.404) (end 131.826 57.32) (width 0.35) (layer B.Cu) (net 9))
 (segment (start 129.37 57.404) (end 131.742 57.404) (width 0.35) (layer B.Cu) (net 9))
 (segment (start 125.476 49.022) (end 126.746 50.292) (width 0.35) (layer B.Cu) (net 9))
 (segment (start 126.746 50.292) (end 126.746 52.578) (width 0.35) (layer B.Cu) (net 9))
 (segment (start 126.746 52.578) (end 127.254 53.086) (width 0.35) (layer B.Cu) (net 9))
 (segment (start 127.254 53.086) (end 131.318 53.086) (width 0.35) (layer B.Cu) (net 9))
 (segment (start 131.318 53.086) (end 131.826 53.594) (width 0.35) (layer B.Cu) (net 9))
 (segment (start 131.826 53.594) (end 131.826 57.32) (width 0.35) (layer B.Cu) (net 9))
 (segment (start 122.936 49.022) (end 125.476 49.022) (width 0.35) (layer B.Cu) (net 9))
 (segment (start 130.302 67.48) (end 136.06 67.48) (width 0.35) (layer B.Cu) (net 10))
 (segment (start 136.06 67.48) (end 137.16 68.58) (width 0.35) (layer B.Cu) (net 10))
 (segment (start 136.048 67.468) (end 137.16 68.58) (width 0.35) (layer F.Cu) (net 10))
 (segment (start 133.73 67.468) (end 136.048 67.468) (width 0.35) (layer F.Cu) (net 10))
 (segment (start 115.888 57.468) (end 114.3 55.88) (width 0.35) (layer F.Cu) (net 11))
 (segment (start 117.73 57.468) (end 115.888 57.468) (width 0.35) (layer F.Cu) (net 11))
 (segment (start 115.348 59.468) (end 114.3 58.42) (width 0.35) (layer F.Cu) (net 12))
 (segment (start 117.73 59.468) (end 115.348 59.468) (width 0.35) (layer F.Cu) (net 12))
 (segment (start 126.83 59.52) (end 126.746 59.436) (width 0.35) (layer B.Cu) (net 12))
 (via (at 126.746 59.436) (size 1) (layers F.Cu B.Cu) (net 12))
 (segment (start 126.746 59.436) (end 126.714 59.468) (width 0.35) (layer F.Cu) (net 12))
 (segment (start 126.714 59.468) (end 124.492 59.468) (width 0.35) (layer F.Cu) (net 12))
 (segment (start 124.492 59.468) (end 124.46 59.468) (width 0.35) (layer F.Cu) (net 12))
 (segment (start 124.46 59.468) (end 117.73 59.468) (width 0.35) (layer F.Cu) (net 12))
 (segment (start 131.826 59.52) (end 126.83 59.52) (width 0.35) (layer B.Cu) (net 12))
 (segment (start 114.808 61.468) (end 114.3 60.96) (width 0.35) (layer F.Cu) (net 13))
 (segment (start 117.73 61.468) (end 114.808 61.468) (width 0.35) (layer F.Cu) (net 13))
 (segment (start 114.332 63.468) (end 114.3 63.5) (width 0.35) (layer F.Cu) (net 14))
 (segment (start 117.73 63.468) (end 114.332 63.468) (width 0.35) (layer F.Cu) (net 14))
 (segment (start 114.872 65.468) (end 114.3 66.04) (width 0.35) (layer F.Cu) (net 15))
 (segment (start 117.73 65.468) (end 114.872 65.468) (width 0.35) (layer F.Cu) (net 15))
 (segment (start 115.412 67.468) (end 114.3 68.58) (width 0.35) (layer F.Cu) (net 16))
 (segment (start 117.73 67.468) (end 115.412 67.468) (width 0.35) (layer F.Cu) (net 16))
 (segment (start 115.952 69.468) (end 114.3 71.12) (width 0.35) (layer F.Cu) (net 17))
 (segment (start 117.73 69.468) (end 115.952 69.468) (width 0.35) (layer F.Cu) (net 17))
 (segment (start 114.46 73.5) (end 114.3 73.66) (width 0.35) (layer F.Cu) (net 18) (status 30))
 (segment (start 120.142 73.66) (end 120.73 73.072) (width 0.35) (layer F.Cu) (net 18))
 (segment (start 120.73 73.072) (end 120.73 71.468) (width 0.35) (layer F.Cu) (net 18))
 (segment (start 114.3 73.66) (end 120.142 73.66) (width 0.35) (layer F.Cu) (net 18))
 (segment (start 121.666 76.2) (end 122.73 75.136) (width 0.35) (layer F.Cu) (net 19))
 (segment (start 122.73 75.136) (end 122.73 71.468) (width 0.35) (layer F.Cu) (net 19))
 (segment (start 114.3 76.2) (end 121.666 76.2) (width 0.35) (layer F.Cu) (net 19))
 (segment (start 130.048 78.74) (end 129.286 79.502) (width 0.35) (layer F.Cu) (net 20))
 (segment (start 129.286 79.502) (end 127.254 79.502) (width 0.35) (layer F.Cu) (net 20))
 (segment (start 127.254 79.502) (end 126.73 78.978) (width 0.35) (layer F.Cu) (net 20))
 (segment (start 126.73 78.978) (end 126.73 71.468) (width 0.35) (layer F.Cu) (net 20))
 (segment (start 137.16 78.74) (end 130.048 78.74) (width 0.35) (layer F.Cu) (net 20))
 (segment (start 128.73 74.882) (end 130.048 76.2) (width 0.35) (layer F.Cu) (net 21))
 (segment (start 130.048 76.2) (end 137.16 76.2) (width 0.35) (layer F.Cu) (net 21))
 (segment (start 128.73 71.468) (end 128.73 74.882) (width 0.35) (layer F.Cu) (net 21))
 (segment (start 131.572 73.66) (end 137.16 73.66) (width 0.35) (layer F.Cu) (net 22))
 (segment (start 130.73 72.818) (end 131.572 73.66) (width 0.35) (layer F.Cu) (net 22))
 (segment (start 130.73 71.468) (end 130.73 72.818) (width 0.35) (layer F.Cu) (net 22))
 (segment (start 120.904 78.74) (end 121.666 79.502) (width 0.35) (layer F.Cu) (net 23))
 (segment (start 121.666 79.502) (end 124.968 79.502) (width 0.35) (layer F.Cu) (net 23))
 (segment (start 124.968 79.502) (end 125.476 78.994) (width 0.35) (layer F.Cu) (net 23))
 (segment (start 125.476 78.994) (end 125.476 75.438) (width 0.35) (layer F.Cu) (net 23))
 (segment (start 125.476 75.438) (end 124.73 74.692) (width 0.35) (layer F.Cu) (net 23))
 (segment (start 124.73 74.692) (end 124.73 71.468) (width 0.35) (layer F.Cu) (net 23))
 (segment (start 114.3 78.74) (end 120.904 78.74) (width 0.35) (layer F.Cu) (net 23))
 (segment (start 136.588 65.468) (end 137.16 66.04) (width 0.35) (layer F.Cu) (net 24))
 (segment (start 133.73 65.468) (end 136.588 65.468) (width 0.35) (layer F.Cu) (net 24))
 (segment (start 137.128 63.468) (end 137.16 63.5) (width 0.35) (layer F.Cu) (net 25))
 (segment (start 133.73 63.468) (end 137.128 63.468) (width 0.35) (layer F.Cu) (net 25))
 (via (at 128.778 63.5) (size 1) (layers F.Cu B.Cu) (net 25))
 (segment (start 128.778 63.5) (end 128.81 63.468) (width 0.35) (layer F.Cu) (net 25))
 (segment (start 128.81 63.468) (end 133.73 63.468) (width 0.35) (layer F.Cu) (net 25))
 (segment (start 125.73 63.5) (end 128.778 63.5) (width 0.35) (layer B.Cu) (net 25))
 (segment (start 136.652 61.468) (end 137.16 60.96) (width 0.35) (layer F.Cu) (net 26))
 (segment (start 133.73 61.468) (end 136.652 61.468) (width 0.35) (layer F.Cu) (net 26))
 (segment (start 136.112 59.468) (end 137.16 58.42) (width 0.35) (layer F.Cu) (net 27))
 (segment (start 133.73 59.468) (end 136.112 59.468) (width 0.35) (layer F.Cu) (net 27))
 (segment (start 135.572 57.468) (end 137.16 55.88) (width 0.35) (layer F.Cu) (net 28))
 (segment (start 133.73 57.468) (end 135.572 57.468) (width 0.35) (layer F.Cu) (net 28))
 (segment (start 128.016 56.642) (end 128.842 57.468) (width 0.35) (layer F.Cu) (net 28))
 (segment (start 128.842 57.468) (end 133.73 57.468) (width 0.35) (layer F.Cu) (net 28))
 (segment (start 128.016 42.926) (end 128.016 56.642) (width 0.35) (layer F.Cu) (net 28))
 (segment (start 133.73 54.23) (end 134.62 53.34) (width 0.35) (layer F.Cu) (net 29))
 (segment (start 134.62 53.34) (end 137.16 53.34) (width 0.35) (layer F.Cu) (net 29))
 (segment (start 133.73 55.468) (end 133.73 54.23) (width 0.35) (layer F.Cu) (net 29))
 (segment (start 125.476 54.61) (end 126.238 55.372) (width 0.35) (layer F.Cu) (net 29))
 (via (at 126.238 55.372) (size 1) (layers F.Cu B.Cu) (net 29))
 (segment (start 126.238 55.372) (end 130.048 55.372) (width 0.35) (layer B.Cu) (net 29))
 (via (at 130.048 55.372) (size 1) (layers F.Cu B.Cu) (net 29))
 (segment (start 130.048 55.372) (end 130.144 55.468) (width 0.35) (layer F.Cu) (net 29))
 (segment (start 130.144 55.468) (end 133.73 55.468) (width 0.35) (layer F.Cu) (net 29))
 (segment (start 125.476 42.926) (end 125.476 54.61) (width 0.35) (layer F.Cu) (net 29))
 (segment (start 124.968 61.468) (end 124.46 60.96) (width 0.35) (layer B.Cu) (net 30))
 (segment (start 124.46 60.96) (end 124.46 57.404) (width 0.35) (layer B.Cu) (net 30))
 (segment (start 128.186 61.468) (end 124.968 61.468) (width 0.35) (layer B.Cu) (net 30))
 (segment (start 125.476 57.404) (end 124.46 57.404) (width 0.35) (layer B.Cu) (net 30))
 (segment (start 127.17 57.404) (end 125.476 57.404) (width 0.35) (layer B.Cu) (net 30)))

